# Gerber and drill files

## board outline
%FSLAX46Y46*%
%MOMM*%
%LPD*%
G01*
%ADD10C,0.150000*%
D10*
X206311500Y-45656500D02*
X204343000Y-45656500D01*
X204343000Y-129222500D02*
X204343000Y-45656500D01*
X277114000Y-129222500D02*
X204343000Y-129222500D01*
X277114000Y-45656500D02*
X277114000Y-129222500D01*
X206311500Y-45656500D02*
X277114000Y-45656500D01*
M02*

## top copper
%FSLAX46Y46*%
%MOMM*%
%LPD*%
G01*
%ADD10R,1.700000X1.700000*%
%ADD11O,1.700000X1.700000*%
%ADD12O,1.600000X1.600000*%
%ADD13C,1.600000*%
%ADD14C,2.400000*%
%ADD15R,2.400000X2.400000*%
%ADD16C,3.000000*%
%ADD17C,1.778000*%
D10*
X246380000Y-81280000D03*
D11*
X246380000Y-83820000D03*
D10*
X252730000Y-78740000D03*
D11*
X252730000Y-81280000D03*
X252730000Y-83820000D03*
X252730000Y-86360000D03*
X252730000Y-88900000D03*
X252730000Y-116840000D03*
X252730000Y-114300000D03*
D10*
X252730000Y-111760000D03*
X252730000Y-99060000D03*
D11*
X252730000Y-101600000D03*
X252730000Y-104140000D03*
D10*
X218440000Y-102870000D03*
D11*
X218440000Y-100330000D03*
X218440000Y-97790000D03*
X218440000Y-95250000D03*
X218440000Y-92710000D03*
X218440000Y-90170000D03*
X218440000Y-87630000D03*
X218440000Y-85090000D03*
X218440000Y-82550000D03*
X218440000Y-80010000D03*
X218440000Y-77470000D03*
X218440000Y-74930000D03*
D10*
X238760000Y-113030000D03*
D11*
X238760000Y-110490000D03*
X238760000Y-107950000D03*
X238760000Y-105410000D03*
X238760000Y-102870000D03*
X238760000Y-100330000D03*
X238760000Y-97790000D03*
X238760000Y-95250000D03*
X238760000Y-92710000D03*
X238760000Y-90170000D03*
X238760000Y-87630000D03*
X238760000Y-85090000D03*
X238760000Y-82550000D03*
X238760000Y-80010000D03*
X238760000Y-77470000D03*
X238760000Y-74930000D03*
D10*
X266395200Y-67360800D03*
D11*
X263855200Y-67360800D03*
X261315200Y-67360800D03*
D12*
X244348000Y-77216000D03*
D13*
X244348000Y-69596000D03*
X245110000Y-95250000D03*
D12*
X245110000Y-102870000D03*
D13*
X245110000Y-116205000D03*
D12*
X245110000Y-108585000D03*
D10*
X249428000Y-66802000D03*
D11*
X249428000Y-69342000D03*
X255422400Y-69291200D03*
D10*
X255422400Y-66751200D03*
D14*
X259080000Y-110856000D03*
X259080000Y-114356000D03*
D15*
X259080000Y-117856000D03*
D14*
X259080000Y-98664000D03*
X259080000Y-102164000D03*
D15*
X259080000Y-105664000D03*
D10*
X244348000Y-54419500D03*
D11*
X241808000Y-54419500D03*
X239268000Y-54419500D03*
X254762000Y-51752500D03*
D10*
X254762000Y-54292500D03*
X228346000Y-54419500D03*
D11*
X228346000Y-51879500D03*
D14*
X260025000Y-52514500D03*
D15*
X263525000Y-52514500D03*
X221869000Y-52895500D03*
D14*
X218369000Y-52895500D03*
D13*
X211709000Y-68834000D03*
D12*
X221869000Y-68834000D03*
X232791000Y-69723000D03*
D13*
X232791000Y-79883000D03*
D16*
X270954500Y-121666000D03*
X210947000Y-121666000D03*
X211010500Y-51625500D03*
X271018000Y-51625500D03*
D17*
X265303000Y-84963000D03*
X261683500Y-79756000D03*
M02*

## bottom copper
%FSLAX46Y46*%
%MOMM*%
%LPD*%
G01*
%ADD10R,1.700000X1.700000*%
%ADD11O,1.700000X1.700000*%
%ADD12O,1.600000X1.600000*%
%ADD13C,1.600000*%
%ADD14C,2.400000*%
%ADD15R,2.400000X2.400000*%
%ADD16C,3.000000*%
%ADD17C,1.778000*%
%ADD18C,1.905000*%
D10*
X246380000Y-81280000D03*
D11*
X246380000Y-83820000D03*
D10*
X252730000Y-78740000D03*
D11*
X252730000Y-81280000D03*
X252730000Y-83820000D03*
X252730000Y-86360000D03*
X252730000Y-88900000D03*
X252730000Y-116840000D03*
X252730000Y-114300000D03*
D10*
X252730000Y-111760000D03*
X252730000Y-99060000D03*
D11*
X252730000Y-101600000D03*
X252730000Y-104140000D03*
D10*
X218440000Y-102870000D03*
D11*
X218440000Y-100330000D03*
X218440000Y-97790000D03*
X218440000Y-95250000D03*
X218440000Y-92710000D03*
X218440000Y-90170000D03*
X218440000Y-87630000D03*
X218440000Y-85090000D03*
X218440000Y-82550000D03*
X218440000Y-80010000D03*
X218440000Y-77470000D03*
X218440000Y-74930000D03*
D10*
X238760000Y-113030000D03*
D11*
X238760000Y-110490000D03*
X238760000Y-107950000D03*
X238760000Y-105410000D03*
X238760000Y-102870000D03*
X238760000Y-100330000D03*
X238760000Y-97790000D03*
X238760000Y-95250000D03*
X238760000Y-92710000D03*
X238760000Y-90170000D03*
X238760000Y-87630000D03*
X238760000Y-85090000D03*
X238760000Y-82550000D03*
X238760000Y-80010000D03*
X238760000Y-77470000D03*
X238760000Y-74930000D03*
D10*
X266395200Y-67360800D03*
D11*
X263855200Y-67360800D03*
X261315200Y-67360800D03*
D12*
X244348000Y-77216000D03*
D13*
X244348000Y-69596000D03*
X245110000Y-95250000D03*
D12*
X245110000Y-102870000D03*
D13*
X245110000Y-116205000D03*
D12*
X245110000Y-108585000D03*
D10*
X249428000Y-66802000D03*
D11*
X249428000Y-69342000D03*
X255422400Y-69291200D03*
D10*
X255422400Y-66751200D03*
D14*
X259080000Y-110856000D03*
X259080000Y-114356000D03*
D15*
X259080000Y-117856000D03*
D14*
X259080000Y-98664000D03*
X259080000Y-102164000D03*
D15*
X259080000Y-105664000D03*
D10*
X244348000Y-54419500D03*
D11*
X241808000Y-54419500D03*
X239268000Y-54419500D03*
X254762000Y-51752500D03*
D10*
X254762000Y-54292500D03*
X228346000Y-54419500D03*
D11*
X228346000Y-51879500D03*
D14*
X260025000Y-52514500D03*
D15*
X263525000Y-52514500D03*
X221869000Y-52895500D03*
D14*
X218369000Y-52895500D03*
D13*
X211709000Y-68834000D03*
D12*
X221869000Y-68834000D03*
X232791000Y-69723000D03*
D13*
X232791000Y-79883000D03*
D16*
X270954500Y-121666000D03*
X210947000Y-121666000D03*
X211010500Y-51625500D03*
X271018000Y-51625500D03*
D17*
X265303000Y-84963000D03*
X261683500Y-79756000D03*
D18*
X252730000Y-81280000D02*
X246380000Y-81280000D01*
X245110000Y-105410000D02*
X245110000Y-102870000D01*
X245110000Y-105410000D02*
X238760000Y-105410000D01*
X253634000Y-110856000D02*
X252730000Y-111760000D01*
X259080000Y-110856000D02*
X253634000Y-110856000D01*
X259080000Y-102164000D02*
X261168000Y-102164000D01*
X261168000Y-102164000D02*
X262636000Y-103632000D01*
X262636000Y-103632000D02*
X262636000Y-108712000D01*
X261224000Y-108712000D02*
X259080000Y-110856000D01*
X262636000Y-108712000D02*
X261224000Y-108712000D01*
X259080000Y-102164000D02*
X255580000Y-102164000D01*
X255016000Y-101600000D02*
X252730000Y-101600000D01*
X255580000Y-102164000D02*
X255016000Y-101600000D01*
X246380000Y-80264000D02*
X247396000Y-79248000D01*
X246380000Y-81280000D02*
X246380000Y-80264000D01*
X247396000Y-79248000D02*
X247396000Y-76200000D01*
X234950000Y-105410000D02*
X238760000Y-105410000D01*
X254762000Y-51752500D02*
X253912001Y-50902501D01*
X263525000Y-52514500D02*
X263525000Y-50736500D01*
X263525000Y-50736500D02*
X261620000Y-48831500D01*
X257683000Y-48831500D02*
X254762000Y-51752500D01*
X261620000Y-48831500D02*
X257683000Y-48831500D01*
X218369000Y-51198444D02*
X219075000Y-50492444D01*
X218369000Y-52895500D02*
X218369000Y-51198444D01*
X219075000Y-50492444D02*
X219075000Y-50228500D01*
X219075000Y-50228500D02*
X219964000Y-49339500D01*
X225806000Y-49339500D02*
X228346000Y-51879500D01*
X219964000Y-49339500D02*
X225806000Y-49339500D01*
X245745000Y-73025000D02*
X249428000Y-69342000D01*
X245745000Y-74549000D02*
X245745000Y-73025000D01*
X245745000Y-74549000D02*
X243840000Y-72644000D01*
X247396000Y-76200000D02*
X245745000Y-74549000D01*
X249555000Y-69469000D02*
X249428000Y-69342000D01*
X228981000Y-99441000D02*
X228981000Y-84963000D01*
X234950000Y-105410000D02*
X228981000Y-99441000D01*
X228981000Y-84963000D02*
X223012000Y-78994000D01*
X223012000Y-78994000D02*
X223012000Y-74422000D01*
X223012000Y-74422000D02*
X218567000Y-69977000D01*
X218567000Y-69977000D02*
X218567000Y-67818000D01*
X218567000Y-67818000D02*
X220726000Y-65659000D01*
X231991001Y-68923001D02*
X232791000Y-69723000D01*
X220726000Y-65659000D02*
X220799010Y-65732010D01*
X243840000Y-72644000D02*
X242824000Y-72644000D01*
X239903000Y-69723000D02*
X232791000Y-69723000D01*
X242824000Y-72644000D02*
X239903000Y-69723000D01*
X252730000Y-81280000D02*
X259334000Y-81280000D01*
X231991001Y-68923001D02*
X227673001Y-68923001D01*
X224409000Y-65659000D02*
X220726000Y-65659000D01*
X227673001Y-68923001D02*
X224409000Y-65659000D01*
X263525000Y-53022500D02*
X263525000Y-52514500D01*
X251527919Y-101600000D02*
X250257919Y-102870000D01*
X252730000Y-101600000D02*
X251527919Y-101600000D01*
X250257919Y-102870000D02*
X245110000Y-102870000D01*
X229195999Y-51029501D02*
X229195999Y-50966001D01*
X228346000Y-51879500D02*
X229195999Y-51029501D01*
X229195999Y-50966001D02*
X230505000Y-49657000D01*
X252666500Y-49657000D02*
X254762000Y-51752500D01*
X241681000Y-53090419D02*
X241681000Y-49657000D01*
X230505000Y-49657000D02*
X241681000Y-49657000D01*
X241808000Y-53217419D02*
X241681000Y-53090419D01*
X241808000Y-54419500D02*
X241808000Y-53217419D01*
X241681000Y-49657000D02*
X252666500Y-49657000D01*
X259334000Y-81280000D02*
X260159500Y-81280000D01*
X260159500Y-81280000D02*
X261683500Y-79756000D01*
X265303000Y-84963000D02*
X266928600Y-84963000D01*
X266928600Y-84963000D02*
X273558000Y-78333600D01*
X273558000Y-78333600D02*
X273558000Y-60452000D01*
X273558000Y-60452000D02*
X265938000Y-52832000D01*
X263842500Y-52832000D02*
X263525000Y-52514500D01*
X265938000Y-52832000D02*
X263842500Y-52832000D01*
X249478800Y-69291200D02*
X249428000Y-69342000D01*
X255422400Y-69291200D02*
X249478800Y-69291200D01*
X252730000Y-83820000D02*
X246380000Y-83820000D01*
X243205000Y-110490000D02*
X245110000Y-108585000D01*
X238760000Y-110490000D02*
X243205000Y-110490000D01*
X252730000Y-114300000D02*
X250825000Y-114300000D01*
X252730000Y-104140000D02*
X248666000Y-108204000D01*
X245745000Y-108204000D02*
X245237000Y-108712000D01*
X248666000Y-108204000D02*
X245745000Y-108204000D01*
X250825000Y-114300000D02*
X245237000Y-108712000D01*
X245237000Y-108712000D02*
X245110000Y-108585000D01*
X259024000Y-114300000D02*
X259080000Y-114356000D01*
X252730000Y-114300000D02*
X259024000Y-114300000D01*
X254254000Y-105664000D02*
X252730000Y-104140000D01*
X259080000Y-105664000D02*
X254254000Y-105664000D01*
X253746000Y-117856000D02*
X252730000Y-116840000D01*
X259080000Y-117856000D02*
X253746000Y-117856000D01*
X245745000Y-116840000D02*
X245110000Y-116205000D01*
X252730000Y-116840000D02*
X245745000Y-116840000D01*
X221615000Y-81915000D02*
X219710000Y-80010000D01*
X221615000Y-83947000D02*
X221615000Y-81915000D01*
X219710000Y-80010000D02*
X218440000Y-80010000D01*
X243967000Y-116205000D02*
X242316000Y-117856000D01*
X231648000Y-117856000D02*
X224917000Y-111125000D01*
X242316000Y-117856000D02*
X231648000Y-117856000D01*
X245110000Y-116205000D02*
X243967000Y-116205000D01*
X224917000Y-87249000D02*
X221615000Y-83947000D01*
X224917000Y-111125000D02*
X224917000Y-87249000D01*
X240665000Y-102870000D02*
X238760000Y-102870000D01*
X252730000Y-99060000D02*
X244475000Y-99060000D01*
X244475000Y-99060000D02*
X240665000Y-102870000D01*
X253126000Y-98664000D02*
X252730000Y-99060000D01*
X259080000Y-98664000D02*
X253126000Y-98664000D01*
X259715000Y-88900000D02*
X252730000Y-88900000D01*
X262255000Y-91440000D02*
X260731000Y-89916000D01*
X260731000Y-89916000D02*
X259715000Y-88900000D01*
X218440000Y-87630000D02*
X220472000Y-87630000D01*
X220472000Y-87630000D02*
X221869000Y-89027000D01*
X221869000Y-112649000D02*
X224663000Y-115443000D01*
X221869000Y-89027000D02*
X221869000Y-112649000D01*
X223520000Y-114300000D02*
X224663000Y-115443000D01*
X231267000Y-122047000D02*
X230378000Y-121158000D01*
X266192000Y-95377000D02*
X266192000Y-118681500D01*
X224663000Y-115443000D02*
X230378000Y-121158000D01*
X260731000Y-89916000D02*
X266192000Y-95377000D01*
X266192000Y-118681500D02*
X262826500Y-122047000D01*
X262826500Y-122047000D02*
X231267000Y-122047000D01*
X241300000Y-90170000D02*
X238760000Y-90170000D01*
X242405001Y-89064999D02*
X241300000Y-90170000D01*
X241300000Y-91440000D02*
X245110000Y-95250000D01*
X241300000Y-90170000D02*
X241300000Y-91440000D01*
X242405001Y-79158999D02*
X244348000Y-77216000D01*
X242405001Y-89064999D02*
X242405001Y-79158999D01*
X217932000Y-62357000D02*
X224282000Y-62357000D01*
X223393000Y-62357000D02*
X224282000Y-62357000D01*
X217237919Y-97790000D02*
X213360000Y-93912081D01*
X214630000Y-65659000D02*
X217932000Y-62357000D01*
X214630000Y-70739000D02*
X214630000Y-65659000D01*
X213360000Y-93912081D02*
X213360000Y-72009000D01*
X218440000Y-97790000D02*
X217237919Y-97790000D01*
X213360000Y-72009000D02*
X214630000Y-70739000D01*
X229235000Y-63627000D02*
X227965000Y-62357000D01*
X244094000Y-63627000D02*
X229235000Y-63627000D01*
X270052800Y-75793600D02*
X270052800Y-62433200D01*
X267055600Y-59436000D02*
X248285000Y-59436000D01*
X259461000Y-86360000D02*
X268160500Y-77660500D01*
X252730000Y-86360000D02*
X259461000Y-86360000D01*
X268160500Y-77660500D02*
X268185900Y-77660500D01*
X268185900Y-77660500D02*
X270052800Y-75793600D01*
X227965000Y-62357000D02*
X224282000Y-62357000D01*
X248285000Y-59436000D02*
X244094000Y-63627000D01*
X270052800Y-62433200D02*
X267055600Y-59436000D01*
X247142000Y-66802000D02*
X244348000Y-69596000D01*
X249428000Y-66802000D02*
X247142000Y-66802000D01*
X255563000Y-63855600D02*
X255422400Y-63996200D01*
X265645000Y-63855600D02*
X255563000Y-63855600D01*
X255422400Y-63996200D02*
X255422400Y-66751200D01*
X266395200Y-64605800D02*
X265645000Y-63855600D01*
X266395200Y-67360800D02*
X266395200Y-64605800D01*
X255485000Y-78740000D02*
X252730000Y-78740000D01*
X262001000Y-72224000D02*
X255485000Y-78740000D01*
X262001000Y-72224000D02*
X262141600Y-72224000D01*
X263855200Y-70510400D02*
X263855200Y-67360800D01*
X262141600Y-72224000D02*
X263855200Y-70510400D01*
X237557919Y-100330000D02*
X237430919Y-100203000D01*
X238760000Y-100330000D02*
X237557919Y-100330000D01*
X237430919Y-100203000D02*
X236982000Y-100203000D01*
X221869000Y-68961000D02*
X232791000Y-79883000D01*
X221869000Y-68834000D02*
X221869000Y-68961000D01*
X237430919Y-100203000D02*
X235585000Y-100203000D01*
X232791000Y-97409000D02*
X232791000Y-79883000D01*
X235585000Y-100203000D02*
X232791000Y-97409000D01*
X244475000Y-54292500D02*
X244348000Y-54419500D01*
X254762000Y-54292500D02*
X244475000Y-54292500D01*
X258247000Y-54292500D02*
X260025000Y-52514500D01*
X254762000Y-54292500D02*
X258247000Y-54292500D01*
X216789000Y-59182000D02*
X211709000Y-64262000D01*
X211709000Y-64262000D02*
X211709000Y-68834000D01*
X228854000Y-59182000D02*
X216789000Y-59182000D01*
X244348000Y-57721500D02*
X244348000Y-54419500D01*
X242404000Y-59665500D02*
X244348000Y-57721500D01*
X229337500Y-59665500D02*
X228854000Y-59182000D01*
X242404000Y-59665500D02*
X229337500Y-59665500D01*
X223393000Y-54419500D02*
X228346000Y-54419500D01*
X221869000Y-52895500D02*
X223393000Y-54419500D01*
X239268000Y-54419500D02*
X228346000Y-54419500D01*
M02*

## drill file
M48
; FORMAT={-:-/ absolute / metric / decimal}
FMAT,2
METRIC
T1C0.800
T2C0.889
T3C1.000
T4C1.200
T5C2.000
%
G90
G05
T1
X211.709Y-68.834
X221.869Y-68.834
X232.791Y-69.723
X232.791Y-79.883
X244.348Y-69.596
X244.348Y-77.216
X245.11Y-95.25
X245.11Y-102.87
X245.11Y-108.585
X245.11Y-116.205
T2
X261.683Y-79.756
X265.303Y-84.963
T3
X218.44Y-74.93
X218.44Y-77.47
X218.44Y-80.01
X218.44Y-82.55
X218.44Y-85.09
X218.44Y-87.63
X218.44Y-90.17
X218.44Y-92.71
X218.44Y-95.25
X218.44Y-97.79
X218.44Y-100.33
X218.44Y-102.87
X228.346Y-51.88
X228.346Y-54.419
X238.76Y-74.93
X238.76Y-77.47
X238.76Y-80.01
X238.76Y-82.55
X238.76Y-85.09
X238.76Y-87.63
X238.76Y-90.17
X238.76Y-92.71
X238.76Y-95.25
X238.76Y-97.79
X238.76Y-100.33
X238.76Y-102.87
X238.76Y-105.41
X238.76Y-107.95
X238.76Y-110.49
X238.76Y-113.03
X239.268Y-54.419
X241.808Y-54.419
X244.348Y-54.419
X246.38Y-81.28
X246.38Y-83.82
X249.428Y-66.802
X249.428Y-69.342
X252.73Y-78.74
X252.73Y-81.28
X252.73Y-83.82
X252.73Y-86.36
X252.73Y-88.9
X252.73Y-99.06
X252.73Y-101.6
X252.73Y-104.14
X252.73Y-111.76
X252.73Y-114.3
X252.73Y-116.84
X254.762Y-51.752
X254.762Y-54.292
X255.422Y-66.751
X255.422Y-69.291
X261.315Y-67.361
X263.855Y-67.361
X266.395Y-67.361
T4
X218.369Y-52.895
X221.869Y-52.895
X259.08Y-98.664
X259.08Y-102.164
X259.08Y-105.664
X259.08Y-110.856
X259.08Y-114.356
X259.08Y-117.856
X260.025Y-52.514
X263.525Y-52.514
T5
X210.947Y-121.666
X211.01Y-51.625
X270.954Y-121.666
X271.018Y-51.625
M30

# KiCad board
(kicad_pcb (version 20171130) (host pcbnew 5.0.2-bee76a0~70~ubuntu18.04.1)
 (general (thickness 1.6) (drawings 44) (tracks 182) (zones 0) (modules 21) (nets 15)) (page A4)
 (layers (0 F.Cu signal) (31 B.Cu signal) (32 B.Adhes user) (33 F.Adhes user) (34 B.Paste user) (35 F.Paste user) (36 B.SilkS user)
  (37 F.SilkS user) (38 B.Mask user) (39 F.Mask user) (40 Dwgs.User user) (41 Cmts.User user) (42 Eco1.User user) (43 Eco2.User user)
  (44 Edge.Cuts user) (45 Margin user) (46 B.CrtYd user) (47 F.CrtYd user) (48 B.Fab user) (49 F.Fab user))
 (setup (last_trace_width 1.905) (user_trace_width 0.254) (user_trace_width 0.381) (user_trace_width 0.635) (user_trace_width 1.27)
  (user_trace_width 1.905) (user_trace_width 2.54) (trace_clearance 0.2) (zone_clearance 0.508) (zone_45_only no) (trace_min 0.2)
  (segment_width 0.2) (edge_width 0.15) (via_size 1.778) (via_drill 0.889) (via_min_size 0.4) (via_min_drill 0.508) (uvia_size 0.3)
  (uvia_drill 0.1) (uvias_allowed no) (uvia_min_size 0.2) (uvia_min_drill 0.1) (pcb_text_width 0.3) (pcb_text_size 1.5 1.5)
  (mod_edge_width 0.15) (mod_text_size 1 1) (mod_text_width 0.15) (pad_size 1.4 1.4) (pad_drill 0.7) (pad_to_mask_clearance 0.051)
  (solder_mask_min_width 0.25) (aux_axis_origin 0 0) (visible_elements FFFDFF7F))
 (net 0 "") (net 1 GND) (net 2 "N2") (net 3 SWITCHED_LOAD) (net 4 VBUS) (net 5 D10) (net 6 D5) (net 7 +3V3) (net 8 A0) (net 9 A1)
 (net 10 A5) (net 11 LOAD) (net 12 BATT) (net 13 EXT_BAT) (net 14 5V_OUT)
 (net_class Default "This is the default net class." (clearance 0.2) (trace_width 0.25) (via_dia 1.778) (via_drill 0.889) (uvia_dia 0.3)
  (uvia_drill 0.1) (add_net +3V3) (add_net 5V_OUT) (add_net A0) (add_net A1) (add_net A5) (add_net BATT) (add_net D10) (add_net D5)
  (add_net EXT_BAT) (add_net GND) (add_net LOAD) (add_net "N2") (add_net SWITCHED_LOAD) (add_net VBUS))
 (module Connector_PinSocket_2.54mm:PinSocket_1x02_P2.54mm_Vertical (layer F.Cu) (at 246.38 81.28)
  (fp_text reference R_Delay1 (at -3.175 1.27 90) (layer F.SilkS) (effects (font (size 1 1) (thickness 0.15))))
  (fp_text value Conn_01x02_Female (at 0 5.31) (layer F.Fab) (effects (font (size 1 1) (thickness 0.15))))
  (pad 1 thru_hole rect (at 0 0) (size 1.7 1.7) (drill 1) (layers *.Cu *.Mask) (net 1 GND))
  (pad 2 thru_hole oval (at 0 2.54) (size 1.7 1.7) (drill 1) (layers *.Cu *.Mask) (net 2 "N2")))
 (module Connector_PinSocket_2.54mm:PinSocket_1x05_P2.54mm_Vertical (layer F.Cu) (at 252.73 78.74)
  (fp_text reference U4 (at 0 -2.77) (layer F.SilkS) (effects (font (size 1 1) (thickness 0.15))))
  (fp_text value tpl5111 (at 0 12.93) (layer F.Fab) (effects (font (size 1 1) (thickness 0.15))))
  (pad 1 thru_hole rect (at 0 0) (size 1.7 1.7) (drill 1) (layers *.Cu *.Mask) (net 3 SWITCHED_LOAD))
  (pad 2 thru_hole oval (at 0 2.54) (size 1.7 1.7) (drill 1) (layers *.Cu *.Mask) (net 1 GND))
  (pad 3 thru_hole oval (at 0 5.08) (size 1.7 1.7) (drill 1) (layers *.Cu *.Mask) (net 2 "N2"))
  (pad 4 thru_hole oval (at 0 7.62) (size 1.7 1.7) (drill 1) (layers *.Cu *.Mask) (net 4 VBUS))
  (pad 5 thru_hole oval (at 0 10.16) (size 1.7 1.7) (drill 1) (layers *.Cu *.Mask) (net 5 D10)))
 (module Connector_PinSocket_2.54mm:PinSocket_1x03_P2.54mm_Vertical (layer F.Cu) (at 252.73 111.76)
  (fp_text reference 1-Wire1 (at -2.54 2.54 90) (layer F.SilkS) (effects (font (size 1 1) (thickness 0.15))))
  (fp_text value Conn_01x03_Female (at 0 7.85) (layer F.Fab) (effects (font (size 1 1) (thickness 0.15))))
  (pad 3 thru_hole oval (at 0 5.08) (size 1.7 1.7) (drill 1) (layers *.Cu *.Mask) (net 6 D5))
  (pad 2 thru_hole oval (at 0 2.54) (size 1.7 1.7) (drill 1) (layers *.Cu *.Mask) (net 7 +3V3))
  (pad 1 thru_hole rect (at 0 0) (size 1.7 1.7) (drill 1) (layers *.Cu *.Mask) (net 1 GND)))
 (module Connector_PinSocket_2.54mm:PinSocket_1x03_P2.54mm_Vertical (layer F.Cu) (at 252.73 99.06)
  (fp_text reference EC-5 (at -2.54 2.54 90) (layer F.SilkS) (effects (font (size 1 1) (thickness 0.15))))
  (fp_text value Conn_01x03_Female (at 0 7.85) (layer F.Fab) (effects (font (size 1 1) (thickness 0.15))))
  (pad 1 thru_hole rect (at 0 0) (size 1.7 1.7) (drill 1) (layers *.Cu *.Mask) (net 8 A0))
  (pad 2 thru_hole oval (at 0 2.54) (size 1.7 1.7) (drill 1) (layers *.Cu *.Mask) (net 1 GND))
  (pad 3 thru_hole oval (at 0 5.08) (size 1.7 1.7) (drill 1) (layers *.Cu *.Mask) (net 7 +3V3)))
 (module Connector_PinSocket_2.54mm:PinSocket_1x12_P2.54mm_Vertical (layer F.Cu) (at 218.44 102.87 180)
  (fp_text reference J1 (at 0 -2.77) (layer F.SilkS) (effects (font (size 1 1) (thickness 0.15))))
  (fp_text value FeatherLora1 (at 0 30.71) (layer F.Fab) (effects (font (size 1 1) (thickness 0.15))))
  (pad 1 thru_hole rect (at 0 0 180) (size 1.7 1.7) (drill 1) (layers *.Cu *.Mask))
  (pad 2 thru_hole oval (at 0 2.54 180) (size 1.7 1.7) (drill 1) (layers *.Cu *.Mask))
  (pad 3 thru_hole oval (at 0 5.08 180) (size 1.7 1.7) (drill 1) (layers *.Cu *.Mask) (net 4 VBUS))
  (pad 4 thru_hole oval (at 0 7.62 180) (size 1.7 1.7) (drill 1) (layers *.Cu *.Mask))
  (pad 5 thru_hole oval (at 0 10.16 180) (size 1.7 1.7) (drill 1) (layers *.Cu *.Mask))
  (pad 6 thru_hole oval (at 0 12.7 180) (size 1.7 1.7) (drill 1) (layers *.Cu *.Mask))
  (pad 7 thru_hole oval (at 0 15.24 180) (size 1.7 1.7) (drill 1) (layers *.Cu *.Mask) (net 5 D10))
  (pad 8 thru_hole oval (at 0 17.78 180) (size 1.7 1.7) (drill 1) (layers *.Cu *.Mask))
  (pad 9 thru_hole oval (at 0 20.32 180) (size 1.7 1.7) (drill 1) (layers *.Cu *.Mask))
  (pad 10 thru_hole oval (at 0 22.86 180) (size 1.7 1.7) (drill 1) (layers *.Cu *.Mask) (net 6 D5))
  (pad 11 thru_hole oval (at 0 25.4 180) (size 1.7 1.7) (drill 1) (layers *.Cu *.Mask))
  (pad 12 thru_hole oval (at 0 27.94 180) (size 1.7 1.7) (drill 1) (layers *.Cu *.Mask)))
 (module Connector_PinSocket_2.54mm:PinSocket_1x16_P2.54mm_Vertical (layer F.Cu) (at 238.76 113.03 180)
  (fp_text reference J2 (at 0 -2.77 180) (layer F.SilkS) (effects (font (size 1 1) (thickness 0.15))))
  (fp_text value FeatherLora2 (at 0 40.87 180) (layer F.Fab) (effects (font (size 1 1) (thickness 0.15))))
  (pad 1 thru_hole rect (at 0 0 180) (size 1.7 1.7) (drill 1) (layers *.Cu *.Mask))
  (pad 2 thru_hole oval (at 0 2.54 180) (size 1.7 1.7) (drill 1) (layers *.Cu *.Mask) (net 7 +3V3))
  (pad 3 thru_hole oval (at 0 5.08 180) (size 1.7 1.7) (drill 1) (layers *.Cu *.Mask))
  (pad 4 thru_hole oval (at 0 7.62 180) (size 1.7 1.7) (drill 1) (layers *.Cu *.Mask) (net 1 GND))
  (pad 5 thru_hole oval (at 0 10.16 180) (size 1.7 1.7) (drill 1) (layers *.Cu *.Mask) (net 8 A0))
  (pad 6 thru_hole oval (at 0 12.7 180) (size 1.7 1.7) (drill 1) (layers *.Cu *.Mask) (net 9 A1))
  (pad 7 thru_hole oval (at 0 15.24 180) (size 1.7 1.7) (drill 1) (layers *.Cu *.Mask))
  (pad 8 thru_hole oval (at 0 17.78 180) (size 1.7 1.7) (drill 1) (layers *.Cu *.Mask))
  (pad 9 thru_hole oval (at 0 20.32 180) (size 1.7 1.7) (drill 1) (layers *.Cu *.Mask))
  (pad 10 thru_hole oval (at 0 22.86 180) (size 1.7 1.7) (drill 1) (layers *.Cu *.Mask) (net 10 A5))
  (pad 11 thru_hole oval (at 0 25.4 180) (size 1.7 1.7) (drill 1) (layers *.Cu *.Mask))
  (pad 12 thru_hole oval (at 0 27.94 180) (size 1.7 1.7) (drill 1) (layers *.Cu *.Mask))
  (pad 13 thru_hole oval (at 0 30.48 180) (size 1.7 1.7) (drill 1) (layers *.Cu *.Mask))
  (pad 14 thru_hole oval (at 0 33.02 180) (size 1.7 1.7) (drill 1) (layers *.Cu *.Mask))
  (pad 15 thru_hole oval (at 0 35.56 180) (size 1.7 1.7) (drill 1) (layers *.Cu *.Mask))
  (pad 16 thru_hole oval (at 0 38.1 180) (size 1.7 1.7) (drill 1) (layers *.Cu *.Mask)))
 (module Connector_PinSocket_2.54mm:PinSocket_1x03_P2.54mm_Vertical (layer F.Cu) (at 266.3952 67.3608 270)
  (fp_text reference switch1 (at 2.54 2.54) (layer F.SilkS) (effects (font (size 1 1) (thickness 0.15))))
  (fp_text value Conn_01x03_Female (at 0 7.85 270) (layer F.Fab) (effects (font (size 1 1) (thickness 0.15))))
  (pad 1 thru_hole rect (at 0 0 270) (size 1.7 1.7) (drill 1) (layers *.Cu *.Mask) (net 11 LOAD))
  (pad 2 thru_hole oval (at 0 2.54 270) (size 1.7 1.7) (drill 1) (layers *.Cu *.Mask) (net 3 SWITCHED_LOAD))
  (pad 3 thru_hole oval (at 0 5.08 270) (size 1.7 1.7) (drill 1) (layers *.Cu *.Mask)))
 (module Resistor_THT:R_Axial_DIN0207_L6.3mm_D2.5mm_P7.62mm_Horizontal (layer F.Cu) (at 244.348 69.596 270)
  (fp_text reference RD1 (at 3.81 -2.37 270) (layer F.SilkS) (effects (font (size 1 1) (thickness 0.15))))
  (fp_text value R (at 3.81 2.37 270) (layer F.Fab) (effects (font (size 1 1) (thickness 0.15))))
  (pad 2 thru_hole oval (at 7.62 0 270) (size 1.6 1.6) (drill 0.8) (layers *.Cu *.Mask) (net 10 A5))
  (pad 1 thru_hole circle (at 0 0 270) (size 1.6 1.6) (drill 0.8) (layers *.Cu *.Mask) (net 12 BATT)))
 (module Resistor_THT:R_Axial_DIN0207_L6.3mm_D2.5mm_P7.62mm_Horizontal (layer F.Cu) (at 245.11 95.25 270)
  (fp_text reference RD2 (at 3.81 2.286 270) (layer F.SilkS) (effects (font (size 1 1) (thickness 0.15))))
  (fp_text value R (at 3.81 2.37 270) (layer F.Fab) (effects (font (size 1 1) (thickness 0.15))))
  (pad 1 thru_hole circle (at 0 0 270) (size 1.6 1.6) (drill 0.8) (layers *.Cu *.Mask) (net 10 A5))
  (pad 2 thru_hole oval (at 7.62 0 270) (size 1.6 1.6) (drill 0.8) (layers *.Cu *.Mask) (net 1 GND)))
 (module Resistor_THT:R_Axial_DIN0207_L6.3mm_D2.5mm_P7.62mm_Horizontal (layer F.Cu) (at 245.11 116.205 90)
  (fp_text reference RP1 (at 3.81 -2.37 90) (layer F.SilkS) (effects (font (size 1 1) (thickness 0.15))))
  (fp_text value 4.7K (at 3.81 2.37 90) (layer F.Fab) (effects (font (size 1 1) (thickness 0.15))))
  (pad 1 thru_hole circle (at 0 0 90) (size 1.6 1.6) (drill 0.8) (layers *.Cu *.Mask) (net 6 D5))
  (pad 2 thru_hole oval (at 7.62 0 90) (size 1.6 1.6) (drill 0.8) (layers *.Cu *.Mask) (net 7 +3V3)))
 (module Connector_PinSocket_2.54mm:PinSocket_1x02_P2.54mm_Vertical (layer F.Cu) (at 249.428 66.802)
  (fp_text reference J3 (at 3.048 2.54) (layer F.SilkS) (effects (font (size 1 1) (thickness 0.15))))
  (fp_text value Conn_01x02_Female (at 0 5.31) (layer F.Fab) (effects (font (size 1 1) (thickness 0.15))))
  (pad 1 thru_hole rect (at 0 0) (size 1.7 1.7) (drill 1) (layers *.Cu *.Mask) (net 12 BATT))
  (pad 2 thru_hole oval (at 0 2.54) (size 1.7 1.7) (drill 1) (layers *.Cu *.Mask) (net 1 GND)))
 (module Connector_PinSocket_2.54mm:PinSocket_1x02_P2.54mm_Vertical (layer F.Cu) (at 255.4224 66.7512)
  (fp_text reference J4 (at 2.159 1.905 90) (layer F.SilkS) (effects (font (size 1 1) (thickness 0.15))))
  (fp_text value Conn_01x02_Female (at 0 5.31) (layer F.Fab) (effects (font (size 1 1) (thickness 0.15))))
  (pad 2 thru_hole oval (at 0 2.54) (size 1.7 1.7) (drill 1) (layers *.Cu *.Mask) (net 1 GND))
  (pad 1 thru_hole rect (at 0 0) (size 1.7 1.7) (drill 1) (layers *.Cu *.Mask) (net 11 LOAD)))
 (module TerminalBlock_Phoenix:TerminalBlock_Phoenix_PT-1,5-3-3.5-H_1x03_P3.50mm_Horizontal (layer F.Cu) (at 259.08 117.856 90)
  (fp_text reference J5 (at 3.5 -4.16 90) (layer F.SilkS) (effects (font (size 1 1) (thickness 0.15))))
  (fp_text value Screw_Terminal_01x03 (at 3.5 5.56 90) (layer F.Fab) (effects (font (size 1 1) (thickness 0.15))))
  (pad 3 thru_hole circle (at 7 0 90) (size 2.4 2.4) (drill 1.2) (layers *.Cu *.Mask) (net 1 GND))
  (pad 2 thru_hole circle (at 3.5 0 90) (size 2.4 2.4) (drill 1.2) (layers *.Cu *.Mask) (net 7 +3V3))
  (pad 1 thru_hole rect (at 0 0 90) (size 2.4 2.4) (drill 1.2) (layers *.Cu *.Mask) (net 6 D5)))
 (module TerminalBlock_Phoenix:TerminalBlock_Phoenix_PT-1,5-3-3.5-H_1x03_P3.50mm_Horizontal (layer F.Cu) (at 259.08 105.664 90)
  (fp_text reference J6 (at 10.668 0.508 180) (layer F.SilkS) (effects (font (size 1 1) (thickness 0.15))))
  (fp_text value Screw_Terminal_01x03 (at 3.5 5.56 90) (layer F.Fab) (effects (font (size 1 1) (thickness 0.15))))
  (pad 3 thru_hole circle (at 7 0 90) (size 2.4 2.4) (drill 1.2) (layers *.Cu *.Mask) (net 8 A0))
  (pad 2 thru_hole circle (at 3.5 0 90) (size 2.4 2.4) (drill 1.2) (layers *.Cu *.Mask) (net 1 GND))
  (pad 1 thru_hole rect (at 0 0 90) (size 2.4 2.4) (drill 1.2) (layers *.Cu *.Mask) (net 7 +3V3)))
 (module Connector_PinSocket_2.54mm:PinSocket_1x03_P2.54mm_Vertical (layer F.Cu) (at 244.348 54.4195 270)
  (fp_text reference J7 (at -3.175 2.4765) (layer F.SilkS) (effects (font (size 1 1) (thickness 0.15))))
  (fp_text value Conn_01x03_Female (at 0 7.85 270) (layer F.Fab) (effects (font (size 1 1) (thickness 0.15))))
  (pad 1 thru_hole rect (at 0 0 270) (size 1.7 1.7) (drill 1) (layers *.Cu *.Mask) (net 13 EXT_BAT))
  (pad 2 thru_hole oval (at 0 2.54 270) (size 1.7 1.7) (drill 1) (layers *.Cu *.Mask) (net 1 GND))
  (pad 3 thru_hole oval (at 0 5.08 270) (size 1.7 1.7) (drill 1) (layers *.Cu *.Mask) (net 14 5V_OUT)))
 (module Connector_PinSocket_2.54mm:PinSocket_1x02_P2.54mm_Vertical (layer F.Cu) (at 254.762 54.2925 180)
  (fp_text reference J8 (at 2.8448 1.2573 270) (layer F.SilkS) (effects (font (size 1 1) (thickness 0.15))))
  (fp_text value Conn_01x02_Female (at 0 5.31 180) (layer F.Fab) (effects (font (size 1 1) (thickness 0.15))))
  (pad 2 thru_hole oval (at 0 2.54 180) (size 1.7 1.7) (drill 1) (layers *.Cu *.Mask) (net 1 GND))
  (pad 1 thru_hole rect (at 0 0 180) (size 1.7 1.7) (drill 1) (layers *.Cu *.Mask) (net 13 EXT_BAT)))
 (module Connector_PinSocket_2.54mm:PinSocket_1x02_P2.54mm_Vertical (layer F.Cu) (at 228.346 54.4195 180)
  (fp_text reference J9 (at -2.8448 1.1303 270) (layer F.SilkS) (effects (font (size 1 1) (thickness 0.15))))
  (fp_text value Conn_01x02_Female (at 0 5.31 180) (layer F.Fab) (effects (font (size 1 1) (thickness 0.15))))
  (pad 1 thru_hole rect (at 0 0 180) (size 1.7 1.7) (drill 1) (layers *.Cu *.Mask) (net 14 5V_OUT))
  (pad 2 thru_hole oval (at 0 2.54 180) (size 1.7 1.7) (drill 1) (layers *.Cu *.Mask) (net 1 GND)))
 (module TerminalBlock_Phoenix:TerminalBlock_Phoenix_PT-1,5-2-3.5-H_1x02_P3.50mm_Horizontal (layer F.Cu) (at 263.525 52.5145 180)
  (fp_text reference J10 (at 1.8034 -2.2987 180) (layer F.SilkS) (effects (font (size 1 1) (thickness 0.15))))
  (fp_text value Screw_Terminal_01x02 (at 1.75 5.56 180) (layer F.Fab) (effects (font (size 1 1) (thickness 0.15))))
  (pad 2 thru_hole circle (at 3.5 0 180) (size 2.4 2.4) (drill 1.2) (layers *.Cu *.Mask) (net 13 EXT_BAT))
  (pad 1 thru_hole rect (at 0 0 180) (size 2.4 2.4) (drill 1.2) (layers *.Cu *.Mask) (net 1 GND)))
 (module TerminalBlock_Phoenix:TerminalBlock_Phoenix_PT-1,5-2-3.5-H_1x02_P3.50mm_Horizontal (layer F.Cu) (at 221.869 52.8955 180)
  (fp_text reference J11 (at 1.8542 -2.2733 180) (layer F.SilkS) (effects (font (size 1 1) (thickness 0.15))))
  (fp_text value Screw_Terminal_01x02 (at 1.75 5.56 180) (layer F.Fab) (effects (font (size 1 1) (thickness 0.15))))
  (pad 1 thru_hole rect (at 0 0 180) (size 2.4 2.4) (drill 1.2) (layers *.Cu *.Mask) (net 14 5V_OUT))
  (pad 2 thru_hole circle (at 3.5 0 180) (size 2.4 2.4) (drill 1.2) (layers *.Cu *.Mask) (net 1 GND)))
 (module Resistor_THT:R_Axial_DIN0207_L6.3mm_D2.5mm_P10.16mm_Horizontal (layer F.Cu) (at 211.709 68.834)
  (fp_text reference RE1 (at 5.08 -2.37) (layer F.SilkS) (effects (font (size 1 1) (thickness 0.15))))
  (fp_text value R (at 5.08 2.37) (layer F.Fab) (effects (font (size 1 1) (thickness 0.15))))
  (pad 1 thru_hole circle (at 0 0) (size 1.6 1.6) (drill 0.8) (layers *.Cu *.Mask) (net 13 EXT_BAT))
  (pad 2 thru_hole oval (at 10.16 0) (size 1.6 1.6) (drill 0.8) (layers *.Cu *.Mask) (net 9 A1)))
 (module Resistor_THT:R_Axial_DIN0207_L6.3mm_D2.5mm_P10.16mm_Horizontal (layer F.Cu) (at 232.791 79.883 90)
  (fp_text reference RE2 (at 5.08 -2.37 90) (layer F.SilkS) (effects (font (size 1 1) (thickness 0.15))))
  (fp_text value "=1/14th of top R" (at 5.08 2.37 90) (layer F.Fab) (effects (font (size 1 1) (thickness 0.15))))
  (pad 2 thru_hole oval (at 10.16 0 90) (size 1.6 1.6) (drill 0.8) (layers *.Cu *.Mask) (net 1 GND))
  (pad 1 thru_hole circle (at 0 0 90) (size 1.6 1.6) (drill 0.8) (layers *.Cu *.Mask) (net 9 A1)))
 (gr_line (start 206.3115 45.6565) (end 204.343 45.6565) (layer Edge.Cuts) (width 0.15))
 (gr_line (start 204.343 129.2225) (end 204.343 45.6565) (layer Edge.Cuts) (width 0.15))
 (gr_line (start 277.114 129.2225) (end 204.343 129.2225) (layer Edge.Cuts) (width 0.15))
 (gr_line (start 277.114 45.6565) (end 277.114 129.2225) (layer Edge.Cuts) (width 0.15))
 (gr_line (start 206.3115 45.6565) (end 277.114 45.6565) (layer Edge.Cuts) (width 0.15))
 (via (at 270.9545 121.666) (size 3) (drill 2) (layers F.Cu B.Cu) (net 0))
 (via (at 210.947 121.666) (size 3) (drill 2) (layers F.Cu B.Cu) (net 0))
 (via (at 211.0105 51.6255) (size 3) (drill 2) (layers F.Cu B.Cu) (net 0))
 (via (at 271.018 51.6255) (size 3) (drill 2) (layers F.Cu B.Cu) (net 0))
 (segment (start 252.73 81.28) (end 246.38 81.28) (width 1.905) (layer B.Cu) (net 1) (status 30))
 (segment (start 245.11 105.41) (end 245.11 102.87) (width 1.905) (layer B.Cu) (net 1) (status 20))
 (segment (start 245.11 105.41) (end 238.76 105.41) (width 1.905) (layer B.Cu) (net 1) (status 20))
 (segment (start 253.634 110.856) (end 252.73 111.76) (width 1.905) (layer B.Cu) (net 1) (status 20))
 (segment (start 259.08 110.856) (end 253.634 110.856) (width 1.905) (layer B.Cu) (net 1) (status 10))
 (segment (start 259.08 102.164) (end 261.168 102.164) (width 1.905) (layer B.Cu) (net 1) (status 10))
 (segment (start 261.168 102.164) (end 262.636 103.632) (width 1.905) (layer B.Cu) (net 1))
 (segment (start 262.636 103.632) (end 262.636 108.712) (width 1.905) (layer B.Cu) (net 1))
 (segment (start 261.224 108.712) (end 259.08 110.856) (width 1.905) (layer B.Cu) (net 1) (status 20))
 (segment (start 262.636 108.712) (end 261.224 108.712) (width 1.905) (layer B.Cu) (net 1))
 (segment (start 259.08 102.164) (end 255.58 102.164) (width 1.905) (layer B.Cu) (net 1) (status 10))
 (segment (start 255.016 101.6) (end 252.73 101.6) (width 1.905) (layer B.Cu) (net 1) (status 20))
 (segment (start 255.58 102.164) (end 255.016 101.6) (width 1.905) (layer B.Cu) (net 1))
 (segment (start 246.38 80.264) (end 247.396 79.248) (width 1.905) (layer B.Cu) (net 1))
 (segment (start 246.38 81.28) (end 246.38 80.264) (width 1.905) (layer B.Cu) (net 1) (status 10))
 (segment (start 247.396 79.248) (end 247.396 76.2) (width 1.905) (layer B.Cu) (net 1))
 (segment (start 234.95 105.41) (end 238.76 105.41) (width 1.905) (layer B.Cu) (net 1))
 (segment (start 254.762 51.7525) (end 253.912001 50.902501) (width 1.905) (layer B.Cu) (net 1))
 (segment (start 263.525 52.5145) (end 263.525 50.7365) (width 1.905) (layer B.Cu) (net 1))
 (segment (start 263.525 50.7365) (end 261.62 48.8315) (width 1.905) (layer B.Cu) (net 1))
 (segment (start 257.683 48.8315) (end 254.762 51.7525) (width 1.905) (layer B.Cu) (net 1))
 (segment (start 261.62 48.8315) (end 257.683 48.8315) (width 1.905) (layer B.Cu) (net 1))
 (segment (start 218.369 51.198444) (end 219.075 50.492444) (width 1.905) (layer B.Cu) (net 1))
 (segment (start 218.369 52.8955) (end 218.369 51.198444) (width 1.905) (layer B.Cu) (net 1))
 (segment (start 219.075 50.492444) (end 219.075 50.2285) (width 1.905) (layer B.Cu) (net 1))
 (segment (start 219.075 50.2285) (end 219.964 49.3395) (width 1.905) (layer B.Cu) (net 1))
 (segment (start 225.806 49.3395) (end 228.346 51.8795) (width 1.905) (layer B.Cu) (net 1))
 (segment (start 219.964 49.3395) (end 225.806 49.3395) (width 1.905) (layer B.Cu) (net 1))
 (segment (start 245.745 73.025) (end 249.428 69.342) (width 1.905) (layer B.Cu) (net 1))
 (segment (start 245.745 74.549) (end 245.745 73.025) (width 1.905) (layer B.Cu) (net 1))
 (segment (start 245.745 74.549) (end 243.84 72.644) (width 1.905) (layer B.Cu) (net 1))
 (segment (start 247.396 76.2) (end 245.745 74.549) (width 1.905) (layer B.Cu) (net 1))
 (segment (start 249.555 69.469) (end 249.428 69.342) (width 1.905) (layer B.Cu) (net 1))
 (segment (start 228.981 99.441) (end 228.981 84.963) (width 1.905) (layer B.Cu) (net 1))
 (segment (start 234.95 105.41) (end 228.981 99.441) (width 1.905) (layer B.Cu) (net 1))
 (segment (start 228.981 84.963) (end 223.012 78.994) (width 1.905) (layer B.Cu) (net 1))
 (segment (start 223.012 78.994) (end 223.012 74.422) (width 1.905) (layer B.Cu) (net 1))
 (segment (start 223.012 74.422) (end 218.567 69.977) (width 1.905) (layer B.Cu) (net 1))
 (segment (start 218.567 69.977) (end 218.567 67.818) (width 1.905) (layer B.Cu) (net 1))
 (segment (start 218.567 67.818) (end 220.726 65.659) (width 1.905) (layer B.Cu) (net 1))
 (segment (start 231.991001 68.923001) (end 232.791 69.723) (width 1.905) (layer B.Cu) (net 1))
 (segment (start 220.726 65.659) (end 220.79901 65.73201) (width 1.905) (layer B.Cu) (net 1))
 (segment (start 243.84 72.644) (end 242.824 72.644) (width 1.905) (layer B.Cu) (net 1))
 (segment (start 239.903 69.723) (end 232.791 69.723) (width 1.905) (layer B.Cu) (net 1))
 (segment (start 242.824 72.644) (end 239.903 69.723) (width 1.905) (layer B.Cu) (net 1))
 (segment (start 252.73 81.28) (end 259.334 81.28) (width 1.905) (layer B.Cu) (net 1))
 (via (at 265.303 84.963) (size 1.778) (drill 0.889) (layers F.Cu B.Cu) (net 1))
 (segment (start 231.991001 68.923001) (end 227.673001 68.923001) (width 1.905) (layer B.Cu) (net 1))
 (segment (start 224.409 65.659) (end 220.726 65.659) (width 1.905) (layer B.Cu) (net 1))
 (segment (start 227.673001 68.923001) (end 224.409 65.659) (width 1.905) (layer B.Cu) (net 1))
 (segment (start 263.525 53.0225) (end 263.525 52.5145) (width 1.905) (layer B.Cu) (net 1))
 (segment (start 251.527919 101.6) (end 250.257919 102.87) (width 1.905) (layer B.Cu) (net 1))
 (segment (start 252.73 101.6) (end 251.527919 101.6) (width 1.905) (layer B.Cu) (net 1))
 (segment (start 250.257919 102.87) (end 245.11 102.87) (width 1.905) (layer B.Cu) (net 1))
 (segment (start 229.195999 51.029501) (end 229.195999 50.966001) (width 1.905) (layer B.Cu) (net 1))
 (segment (start 228.346 51.8795) (end 229.195999 51.029501) (width 1.905) (layer B.Cu) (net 1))
 (segment (start 229.195999 50.966001) (end 230.505 49.657) (width 1.905) (layer B.Cu) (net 1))
 (segment (start 252.6665 49.657) (end 254.762 51.7525) (width 1.905) (layer B.Cu) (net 1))
 (segment (start 241.681 53.090419) (end 241.681 49.657) (width 1.905) (layer B.Cu) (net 1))
 (segment (start 230.505 49.657) (end 241.681 49.657) (width 1.905) (layer B.Cu) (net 1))
 (segment (start 241.808 53.217419) (end 241.681 53.090419) (width 1.905) (layer B.Cu) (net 1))
 (segment (start 241.808 54.4195) (end 241.808 53.217419) (width 1.905) (layer B.Cu) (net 1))
 (segment (start 241.681 49.657) (end 252.6665 49.657) (width 1.905) (layer B.Cu) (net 1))
 (via (at 261.6835 79.756) (size 1.778) (drill 0.889) (layers F.Cu B.Cu) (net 1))
 (segment (start 259.334 81.28) (end 260.1595 81.28) (width 1.905) (layer B.Cu) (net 1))
 (segment (start 260.1595 81.28) (end 261.6835 79.756) (width 1.905) (layer B.Cu) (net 1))
 (segment (start 265.303 84.963) (end 266.9286 84.963) (width 1.905) (layer B.Cu) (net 1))
 (segment (start 266.9286 84.963) (end 273.558 78.3336) (width 1.905) (layer B.Cu) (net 1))
 (segment (start 273.558 78.3336) (end 273.558 60.452) (width 1.905) (layer B.Cu) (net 1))
 (segment (start 273.558 60.452) (end 265.938 52.832) (width 1.905) (layer B.Cu) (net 1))
 (segment (start 263.8425 52.832) (end 263.525 52.5145) (width 1.905) (layer B.Cu) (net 1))
 (segment (start 265.938 52.832) (end 263.8425 52.832) (width 1.905) (layer B.Cu) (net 1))
 (segment (start 249.4788 69.2912) (end 249.428 69.342) (width 1.905) (layer B.Cu) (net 1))
 (segment (start 255.4224 69.2912) (end 249.4788 69.2912) (width 1.905) (layer B.Cu) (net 1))
 (segment (start 252.73 83.82) (end 246.38 83.82) (width 1.905) (layer B.Cu) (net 2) (status 30))
 (segment (start 243.205 110.49) (end 245.11 108.585) (width 1.905) (layer B.Cu) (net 7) (status 20))
 (segment (start 238.76 110.49) (end 243.205 110.49) (width 1.905) (layer B.Cu) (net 7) (status 10))
 (segment (start 252.73 114.3) (end 250.825 114.3) (width 1.905) (layer B.Cu) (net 7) (status 10))
 (segment (start 252.73 104.14) (end 248.666 108.204) (width 1.905) (layer B.Cu) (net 7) (status 10))
 (segment (start 245.745 108.204) (end 245.237 108.712) (width 1.905) (layer B.Cu) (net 7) (status 30))
 (segment (start 248.666 108.204) (end 245.745 108.204) (width 1.905) (layer B.Cu) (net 7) (status 20))
 (segment (start 250.825 114.3) (end 245.237 108.712) (width 1.905) (layer B.Cu) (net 7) (status 20))
 (segment (start 245.237 108.712) (end 245.11 108.585) (width 1.905) (layer B.Cu) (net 7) (status 30))
 (segment (start 259.024 114.3) (end 259.08 114.356) (width 1.905) (layer B.Cu) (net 7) (status 30))
 (segment (start 252.73 114.3) (end 259.024 114.3) (width 1.905) (layer B.Cu) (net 7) (status 30))
 (segment (start 254.254 105.664) (end 252.73 104.14) (width 1.905) (layer B.Cu) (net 7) (status 20))
 (segment (start 259.08 105.664) (end 254.254 105.664) (width 1.905) (layer B.Cu) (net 7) (status 10))
 (segment (start 253.746 117.856) (end 252.73 116.84) (width 1.905) (layer B.Cu) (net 6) (status 20))
 (segment (start 259.08 117.856) (end 253.746 117.856) (width 1.905) (layer B.Cu) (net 6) (status 10))
 (segment (start 245.745 116.84) (end 245.11 116.205) (width 1.905) (layer B.Cu) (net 6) (status 20))
 (segment (start 252.73 116.84) (end 245.745 116.84) (width 1.905) (layer B.Cu) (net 6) (status 10))
 (segment (start 221.615 81.915) (end 219.71 80.01) (width 1.905) (layer B.Cu) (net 6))
 (segment (start 221.615 83.947) (end 221.615 81.915) (width 1.905) (layer B.Cu) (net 6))
 (segment (start 219.71 80.01) (end 218.44 80.01) (width 1.905) (layer B.Cu) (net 6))
 (segment (start 243.967 116.205) (end 242.316 117.856) (width 1.905) (layer B.Cu) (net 6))
 (segment (start 231.648 117.856) (end 224.917 111.125) (width 1.905) (layer B.Cu) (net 6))
 (segment (start 242.316 117.856) (end 231.648 117.856) (width 1.905) (layer B.Cu) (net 6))
 (segment (start 245.11 116.205) (end 243.967 116.205) (width 1.905) (layer B.Cu) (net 6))
 (segment (start 224.917 87.249) (end 221.615 83.947) (width 1.905) (layer B.Cu) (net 6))
 (segment (start 224.917 111.125) (end 224.917 87.249) (width 1.905) (layer B.Cu) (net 6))
 (segment (start 240.665 102.87) (end 238.76 102.87) (width 1.905) (layer B.Cu) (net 8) (status 20))
 (segment (start 252.73 99.06) (end 244.475 99.06) (width 1.905) (layer B.Cu) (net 8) (status 10))
 (segment (start 244.475 99.06) (end 240.665 102.87) (width 1.905) (layer B.Cu) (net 8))
 (segment (start 253.126 98.664) (end 252.73 99.06) (width 1.905) (layer B.Cu) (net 8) (status 30))
 (segment (start 259.08 98.664) (end 253.126 98.664) (width 1.905) (layer B.Cu) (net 8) (status 30))
 (segment (start 259.715 88.9) (end 252.73 88.9) (width 1.905) (layer B.Cu) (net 5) (status 20))
 (segment (start 262.255 91.44) (end 260.731 89.916) (width 1.905) (layer B.Cu) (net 5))
 (segment (start 260.731 89.916) (end 259.715 88.9) (width 1.905) (layer B.Cu) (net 5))
 (segment (start 218.44 87.63) (end 220.472 87.63) (width 1.905) (layer B.Cu) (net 5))
 (segment (start 220.472 87.63) (end 221.869 89.027) (width 1.905) (layer B.Cu) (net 5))
 (segment (start 221.869 112.649) (end 224.663 115.443) (width 1.905) (layer B.Cu) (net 5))
 (segment (start 221.869 89.027) (end 221.869 112.649) (width 1.905) (layer B.Cu) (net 5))
 (segment (start 223.52 114.3) (end 224.663 115.443) (width 1.905) (layer B.Cu) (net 5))
 (segment (start 231.267 122.047) (end 230.378 121.158) (width 1.905) (layer B.Cu) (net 5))
 (segment (start 266.192 95.377) (end 266.192 118.6815) (width 1.905) (layer B.Cu) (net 5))
 (segment (start 224.663 115.443) (end 230.378 121.158) (width 1.905) (layer B.Cu) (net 5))
 (segment (start 260.731 89.916) (end 266.192 95.377) (width 1.905) (layer B.Cu) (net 5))
 (segment (start 266.192 118.6815) (end 262.8265 122.047) (width 1.905) (layer B.Cu) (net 5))
 (segment (start 262.8265 122.047) (end 231.267 122.047) (width 1.905) (layer B.Cu) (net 5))
 (segment (start 241.3 90.17) (end 238.76 90.17) (width 1.905) (layer B.Cu) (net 10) (status 20))
 (segment (start 242.405001 89.064999) (end 241.3 90.17) (width 1.905) (layer B.Cu) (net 10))
 (segment (start 241.3 91.44) (end 245.11 95.25) (width 1.905) (layer B.Cu) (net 10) (status 20))
 (segment (start 241.3 90.17) (end 241.3 91.44) (width 1.905) (layer B.Cu) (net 10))
 (segment (start 242.405001 79.158999) (end 244.348 77.216) (width 1.905) (layer B.Cu) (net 10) (status 20))
 (segment (start 242.405001 89.064999) (end 242.405001 79.158999) (width 1.905) (layer B.Cu) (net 10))
 (segment (start 217.932 62.357) (end 224.282 62.357) (width 1.905) (layer B.Cu) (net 4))
 (segment (start 223.393 62.357) (end 224.282 62.357) (width 1.905) (layer B.Cu) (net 4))
 (segment (start 217.237919 97.79) (end 213.36 93.912081) (width 1.905) (layer B.Cu) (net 4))
 (segment (start 214.63 65.659) (end 217.932 62.357) (width 1.905) (layer B.Cu) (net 4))
 (segment (start 214.63 70.739) (end 214.63 65.659) (width 1.905) (layer B.Cu) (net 4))
 (segment (start 213.36 93.912081) (end 213.36 72.009) (width 1.905) (layer B.Cu) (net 4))
 (segment (start 218.44 97.79) (end 217.237919 97.79) (width 1.905) (layer B.Cu) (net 4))
 (segment (start 213.36 72.009) (end 214.63 70.739) (width 1.905) (layer B.Cu) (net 4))
 (segment (start 229.235 63.627) (end 227.965 62.357) (width 1.905) (layer B.Cu) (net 4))
 (segment (start 244.094 63.627) (end 229.235 63.627) (width 1.905) (layer B.Cu) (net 4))
 (segment (start 270.0528 75.7936) (end 270.0528 62.4332) (width 1.905) (layer B.Cu) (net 4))
 (segment (start 267.0556 59.436) (end 248.285 59.436) (width 1.905) (layer B.Cu) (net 4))
 (segment (start 259.461 86.36) (end 268.1605 77.6605) (width 1.905) (layer B.Cu) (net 4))
 (segment (start 252.73 86.36) (end 259.461 86.36) (width 1.905) (layer B.Cu) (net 4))
 (segment (start 268.1605 77.6605) (end 268.1859 77.6605) (width 1.905) (layer B.Cu) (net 4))
 (segment (start 268.1859 77.6605) (end 270.0528 75.7936) (width 1.905) (layer B.Cu) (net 4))
 (segment (start 227.965 62.357) (end 224.282 62.357) (width 1.905) (layer B.Cu) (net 4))
 (segment (start 248.285 59.436) (end 244.094 63.627) (width 1.905) (layer B.Cu) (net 4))
 (segment (start 270.0528 62.4332) (end 267.0556 59.436) (width 1.905) (layer B.Cu) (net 4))
 (segment (start 247.142 66.802) (end 244.348 69.596) (width 1.905) (layer B.Cu) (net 12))
 (segment (start 249.428 66.802) (end 247.142 66.802) (width 1.905) (layer B.Cu) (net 12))
 (segment (start 255.563 63.8556) (end 255.4224 63.9962) (width 1.905) (layer B.Cu) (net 11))
 (segment (start 265.645 63.8556) (end 255.563 63.8556) (width 1.905) (layer B.Cu) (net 11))
 (segment (start 255.4224 63.9962) (end 255.4224 66.7512) (width 1.905) (layer B.Cu) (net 11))
 (segment (start 266.3952 64.6058) (end 265.645 63.8556) (width 1.905) (layer B.Cu) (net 11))
 (segment (start 266.3952 67.3608) (end 266.3952 64.6058) (width 1.905) (layer B.Cu) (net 11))
 (segment (start 255.485 78.74) (end 252.73 78.74) (width 1.905) (layer B.Cu) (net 3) (status 20))
 (segment (start 262.001 72.224) (end 255.485 78.74) (width 1.905) (layer B.Cu) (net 3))
 (segment (start 262.001 72.224) (end 262.1416 72.224) (width 1.905) (layer B.Cu) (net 3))
 (segment (start 263.8552 70.5104) (end 263.8552 67.3608) (width 1.905) (layer B.Cu) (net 3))
 (segment (start 262.1416 72.224) (end 263.8552 70.5104) (width 1.905) (layer B.Cu) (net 3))
 (segment (start 237.557919 100.33) (end 237.430919 100.203) (width 1.905) (layer B.Cu) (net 9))
 (segment (start 238.76 100.33) (end 237.557919 100.33) (width 1.905) (layer B.Cu) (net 9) (status 10))
 (segment (start 237.430919 100.203) (end 236.982 100.203) (width 1.905) (layer B.Cu) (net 9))
 (segment (start 221.869 68.961) (end 232.791 79.883) (width 1.905) (layer B.Cu) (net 9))
 (segment (start 221.869 68.834) (end 221.869 68.961) (width 1.905) (layer B.Cu) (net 9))
 (segment (start 237.430919 100.203) (end 235.585 100.203) (width 1.905) (layer B.Cu) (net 9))
 (segment (start 232.791 97.409) (end 232.791 79.883) (width 1.905) (layer B.Cu) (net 9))
 (segment (start 235.585 100.203) (end 232.791 97.409) (width 1.905) (layer B.Cu) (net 9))
 (segment (start 244.475 54.2925) (end 244.348 54.4195) (width 1.905) (layer B.Cu) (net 13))
 (segment (start 254.762 54.2925) (end 244.475 54.2925) (width 1.905) (layer B.Cu) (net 13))
 (segment (start 258.247 54.2925) (end 260.025 52.5145) (width 1.905) (layer B.Cu) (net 13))
 (segment (start 254.762 54.2925) (end 258.247 54.2925) (width 1.905) (layer B.Cu) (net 13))
 (segment (start 216.789 59.182) (end 211.709 64.262) (width 1.905) (layer B.Cu) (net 13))
 (segment (start 211.709 64.262) (end 211.709 68.834) (width 1.905) (layer B.Cu) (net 13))
 (segment (start 228.854 59.182) (end 216.789 59.182) (width 1.905) (layer B.Cu) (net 13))
 (segment (start 244.348 57.7215) (end 244.348 54.4195) (width 1.905) (layer B.Cu) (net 13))
 (segment (start 242.404 59.6655) (end 244.348 57.7215) (width 1.905) (layer B.Cu) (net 13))
 (segment (start 229.3375 59.6655) (end 228.854 59.182) (width 1.905) (layer B.Cu) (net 13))
 (segment (start 242.404 59.6655) (end 229.3375 59.6655) (width 1.905) (layer B.Cu) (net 13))
 (segment (start 223.393 54.4195) (end 228.346 54.4195) (width 1.905) (layer B.Cu) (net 14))
 (segment (start 221.869 52.8955) (end 223.393 54.4195) (width 1.905) (layer B.Cu) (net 14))
 (segment (start 239.268 54.4195) (end 228.346 54.4195) (width 1.905) (layer B.Cu) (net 14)))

